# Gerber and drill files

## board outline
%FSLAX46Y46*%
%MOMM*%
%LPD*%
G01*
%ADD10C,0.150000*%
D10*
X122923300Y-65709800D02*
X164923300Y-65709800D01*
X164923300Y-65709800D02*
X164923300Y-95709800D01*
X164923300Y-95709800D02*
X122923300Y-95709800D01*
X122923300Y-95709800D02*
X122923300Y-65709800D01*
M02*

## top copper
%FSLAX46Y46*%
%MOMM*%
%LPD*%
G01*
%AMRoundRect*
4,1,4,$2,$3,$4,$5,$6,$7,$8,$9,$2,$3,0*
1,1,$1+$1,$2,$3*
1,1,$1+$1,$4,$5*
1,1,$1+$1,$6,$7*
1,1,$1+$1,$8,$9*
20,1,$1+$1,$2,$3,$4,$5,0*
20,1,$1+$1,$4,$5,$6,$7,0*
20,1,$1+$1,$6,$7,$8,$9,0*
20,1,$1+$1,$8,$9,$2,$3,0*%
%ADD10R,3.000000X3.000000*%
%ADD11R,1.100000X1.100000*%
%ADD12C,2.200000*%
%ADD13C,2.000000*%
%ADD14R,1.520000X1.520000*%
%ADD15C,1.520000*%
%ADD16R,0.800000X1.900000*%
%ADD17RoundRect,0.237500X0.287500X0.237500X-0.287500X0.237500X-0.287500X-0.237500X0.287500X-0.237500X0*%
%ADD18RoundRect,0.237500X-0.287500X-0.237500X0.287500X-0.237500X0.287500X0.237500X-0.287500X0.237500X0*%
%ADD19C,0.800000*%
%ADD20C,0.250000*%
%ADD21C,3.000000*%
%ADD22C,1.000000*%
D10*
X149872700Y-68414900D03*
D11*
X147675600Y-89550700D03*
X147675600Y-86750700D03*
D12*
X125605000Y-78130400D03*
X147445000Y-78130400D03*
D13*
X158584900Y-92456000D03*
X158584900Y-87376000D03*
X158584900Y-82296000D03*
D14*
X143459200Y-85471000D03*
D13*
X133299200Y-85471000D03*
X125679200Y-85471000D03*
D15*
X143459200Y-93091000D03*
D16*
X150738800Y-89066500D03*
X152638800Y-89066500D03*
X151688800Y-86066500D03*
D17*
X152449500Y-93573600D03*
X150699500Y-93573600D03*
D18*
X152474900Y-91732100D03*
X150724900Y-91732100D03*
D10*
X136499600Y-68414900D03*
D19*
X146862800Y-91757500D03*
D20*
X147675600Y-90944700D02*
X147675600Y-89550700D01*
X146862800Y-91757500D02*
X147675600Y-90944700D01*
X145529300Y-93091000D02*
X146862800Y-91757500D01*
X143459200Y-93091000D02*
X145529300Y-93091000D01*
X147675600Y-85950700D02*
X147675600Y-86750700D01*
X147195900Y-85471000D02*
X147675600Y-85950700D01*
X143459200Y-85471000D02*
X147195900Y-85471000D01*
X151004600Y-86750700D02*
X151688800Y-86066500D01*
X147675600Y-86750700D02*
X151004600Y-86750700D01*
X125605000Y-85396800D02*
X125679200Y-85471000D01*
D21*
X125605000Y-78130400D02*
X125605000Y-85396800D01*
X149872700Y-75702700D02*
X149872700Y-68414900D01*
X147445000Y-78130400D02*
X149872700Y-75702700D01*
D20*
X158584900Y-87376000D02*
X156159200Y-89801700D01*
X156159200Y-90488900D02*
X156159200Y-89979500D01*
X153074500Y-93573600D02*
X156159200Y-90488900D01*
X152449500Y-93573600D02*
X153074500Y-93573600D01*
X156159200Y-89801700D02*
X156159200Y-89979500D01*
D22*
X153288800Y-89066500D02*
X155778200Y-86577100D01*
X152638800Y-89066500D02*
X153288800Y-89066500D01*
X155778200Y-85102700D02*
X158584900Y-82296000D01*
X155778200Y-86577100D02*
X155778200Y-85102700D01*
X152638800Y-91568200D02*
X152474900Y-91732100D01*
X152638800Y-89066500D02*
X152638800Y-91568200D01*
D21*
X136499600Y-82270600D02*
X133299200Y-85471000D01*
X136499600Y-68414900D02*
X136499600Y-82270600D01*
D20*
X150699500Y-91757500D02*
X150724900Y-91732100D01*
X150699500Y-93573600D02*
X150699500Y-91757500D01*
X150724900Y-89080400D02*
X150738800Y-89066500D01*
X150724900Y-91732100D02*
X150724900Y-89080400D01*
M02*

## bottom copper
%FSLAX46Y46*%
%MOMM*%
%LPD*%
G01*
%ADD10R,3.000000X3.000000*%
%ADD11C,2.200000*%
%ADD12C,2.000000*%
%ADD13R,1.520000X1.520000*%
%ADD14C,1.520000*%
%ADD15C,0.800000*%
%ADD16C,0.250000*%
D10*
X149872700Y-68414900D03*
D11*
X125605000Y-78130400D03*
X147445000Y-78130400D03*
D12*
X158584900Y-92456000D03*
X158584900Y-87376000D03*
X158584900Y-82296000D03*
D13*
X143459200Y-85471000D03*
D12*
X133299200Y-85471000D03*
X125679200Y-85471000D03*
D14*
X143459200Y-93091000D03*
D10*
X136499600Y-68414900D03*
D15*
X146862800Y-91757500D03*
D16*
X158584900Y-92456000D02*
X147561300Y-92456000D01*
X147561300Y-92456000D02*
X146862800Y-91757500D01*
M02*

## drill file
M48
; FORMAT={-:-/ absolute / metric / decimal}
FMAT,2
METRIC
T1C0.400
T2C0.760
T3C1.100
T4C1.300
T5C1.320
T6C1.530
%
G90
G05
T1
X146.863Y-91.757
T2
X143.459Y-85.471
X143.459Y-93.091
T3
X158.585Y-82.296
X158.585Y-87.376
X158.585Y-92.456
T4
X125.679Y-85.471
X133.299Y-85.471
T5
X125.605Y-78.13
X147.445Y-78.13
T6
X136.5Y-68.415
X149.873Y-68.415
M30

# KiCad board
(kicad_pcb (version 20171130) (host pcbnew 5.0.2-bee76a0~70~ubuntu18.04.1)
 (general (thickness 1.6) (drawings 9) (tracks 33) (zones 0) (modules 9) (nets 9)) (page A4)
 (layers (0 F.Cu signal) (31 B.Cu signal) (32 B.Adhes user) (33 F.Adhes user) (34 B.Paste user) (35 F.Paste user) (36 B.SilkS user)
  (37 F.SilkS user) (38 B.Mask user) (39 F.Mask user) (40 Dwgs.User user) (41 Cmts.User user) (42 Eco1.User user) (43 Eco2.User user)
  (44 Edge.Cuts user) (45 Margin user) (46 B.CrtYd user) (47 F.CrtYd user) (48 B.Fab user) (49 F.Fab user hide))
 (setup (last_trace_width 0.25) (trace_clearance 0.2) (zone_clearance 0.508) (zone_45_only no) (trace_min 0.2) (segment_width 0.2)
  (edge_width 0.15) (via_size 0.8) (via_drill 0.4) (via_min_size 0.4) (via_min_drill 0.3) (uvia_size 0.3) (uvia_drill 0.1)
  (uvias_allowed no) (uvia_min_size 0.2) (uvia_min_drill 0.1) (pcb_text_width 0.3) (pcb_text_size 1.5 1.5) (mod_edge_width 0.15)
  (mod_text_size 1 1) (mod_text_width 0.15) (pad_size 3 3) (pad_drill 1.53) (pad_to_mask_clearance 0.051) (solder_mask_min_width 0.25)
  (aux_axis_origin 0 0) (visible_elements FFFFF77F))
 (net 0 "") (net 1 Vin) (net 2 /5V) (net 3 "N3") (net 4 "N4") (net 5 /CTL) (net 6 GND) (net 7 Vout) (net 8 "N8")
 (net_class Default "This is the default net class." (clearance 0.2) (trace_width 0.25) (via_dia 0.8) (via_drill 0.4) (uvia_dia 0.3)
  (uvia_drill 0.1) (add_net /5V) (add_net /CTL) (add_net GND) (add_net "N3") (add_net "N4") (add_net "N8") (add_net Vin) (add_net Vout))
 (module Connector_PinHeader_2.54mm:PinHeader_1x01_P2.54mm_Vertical (layer F.Cu) (at 149.8727 68.4149)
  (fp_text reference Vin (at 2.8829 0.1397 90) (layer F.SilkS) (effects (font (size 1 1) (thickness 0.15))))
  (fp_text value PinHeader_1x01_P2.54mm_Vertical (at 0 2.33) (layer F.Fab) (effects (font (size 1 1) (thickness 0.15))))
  (pad 1 thru_hole rect (at 0 0) (size 3 3) (drill 1.53) (layers *.Cu *.Mask) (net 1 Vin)))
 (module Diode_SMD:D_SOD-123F (layer F.Cu) (at 147.6756 88.1507 90)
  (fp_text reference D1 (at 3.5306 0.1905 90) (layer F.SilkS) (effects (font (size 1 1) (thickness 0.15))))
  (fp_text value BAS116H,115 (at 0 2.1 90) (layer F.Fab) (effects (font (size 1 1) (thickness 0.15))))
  (pad 1 smd rect (at -1.4 0 90) (size 1.1 1.1) (layers F.Cu F.Paste F.Mask) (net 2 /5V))
  (pad 2 smd rect (at 1.4 0 90) (size 1.1 1.1) (layers F.Cu F.Paste F.Mask) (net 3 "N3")))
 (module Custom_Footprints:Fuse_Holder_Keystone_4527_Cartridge (layer F.Cu) (at 136.525 78.1304)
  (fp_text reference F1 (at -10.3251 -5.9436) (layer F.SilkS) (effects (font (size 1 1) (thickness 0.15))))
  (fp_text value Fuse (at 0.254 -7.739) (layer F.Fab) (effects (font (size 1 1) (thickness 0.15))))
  (pad 1 thru_hole circle (at -10.92 0) (size 2.2 2.2) (drill 1.32) (layers *.Cu *.Mask) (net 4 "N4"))
  (pad 2 thru_hole circle (at 10.92 0) (size 2.2 2.2) (drill 1.32) (layers *.Cu *.Mask) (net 1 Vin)))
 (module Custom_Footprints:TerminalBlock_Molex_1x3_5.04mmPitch (layer F.Cu) (at 158.5849 87.376 90)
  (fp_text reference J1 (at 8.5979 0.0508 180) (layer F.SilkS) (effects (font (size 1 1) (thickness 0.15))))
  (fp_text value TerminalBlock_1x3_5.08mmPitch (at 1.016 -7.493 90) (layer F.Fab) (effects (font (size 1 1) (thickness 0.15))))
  (pad 1 thru_hole circle (at -5.08 0 90) (size 2 2) (drill 1.1) (layers *.Cu *.Mask) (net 2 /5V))
  (pad 2 thru_hole circle (at 0 0 90) (size 2 2) (drill 1.1) (layers *.Cu *.Mask) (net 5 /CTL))
  (pad 3 thru_hole circle (at 5.08 0 90) (size 2 2) (drill 1.1) (layers *.Cu *.Mask) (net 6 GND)))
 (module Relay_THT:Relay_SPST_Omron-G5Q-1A (layer F.Cu) (at 143.4592 85.471 180)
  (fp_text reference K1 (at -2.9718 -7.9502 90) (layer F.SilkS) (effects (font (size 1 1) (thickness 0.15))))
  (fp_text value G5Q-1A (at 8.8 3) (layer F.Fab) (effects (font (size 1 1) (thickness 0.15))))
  (pad 1 thru_hole rect (at 0 0) (size 1.52 1.52) (drill 0.76) (layers *.Cu *.Mask) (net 3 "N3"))
  (pad 2 thru_hole circle (at 10.16 0) (size 2 2) (drill 1.3) (layers *.Cu *.Mask) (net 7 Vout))
  (pad 3 thru_hole circle (at 17.78 0) (size 2 2) (drill 1.3) (layers *.Cu *.Mask) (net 4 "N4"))
  (pad 5 thru_hole circle (at 0 -7.62) (size 1.52 1.52) (drill 0.76) (layers *.Cu *.Mask) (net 2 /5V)))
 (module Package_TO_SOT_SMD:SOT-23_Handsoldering (layer F.Cu) (at 151.6888 87.5665 90)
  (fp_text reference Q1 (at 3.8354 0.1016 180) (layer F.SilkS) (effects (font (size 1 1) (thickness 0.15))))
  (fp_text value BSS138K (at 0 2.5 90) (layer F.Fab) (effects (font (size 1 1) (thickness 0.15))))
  (pad 1 smd rect (at -1.5 -0.95 90) (size 1.9 0.8) (layers F.Cu F.Paste F.Mask) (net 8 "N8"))
  (pad 2 smd rect (at -1.5 0.95 90) (size 1.9 0.8) (layers F.Cu F.Paste F.Mask) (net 6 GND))
  (pad 3 smd rect (at 1.5 0 90) (size 1.9 0.8) (layers F.Cu F.Paste F.Mask) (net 3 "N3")))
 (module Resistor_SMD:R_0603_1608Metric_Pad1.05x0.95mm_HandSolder (layer F.Cu) (at 151.5745 93.5736 180)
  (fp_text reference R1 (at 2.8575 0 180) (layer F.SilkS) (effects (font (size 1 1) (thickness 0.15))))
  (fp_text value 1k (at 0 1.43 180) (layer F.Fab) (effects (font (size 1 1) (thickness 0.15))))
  (pad 1 smd roundrect (at -0.875 0 180) (size 1.05 0.95) (layers F.Cu F.Paste F.Mask) (roundrect_rratio 0.25) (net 5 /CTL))
  (pad 2 smd roundrect (at 0.875 0 180) (size 1.05 0.95) (layers F.Cu F.Paste F.Mask) (roundrect_rratio 0.25) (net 8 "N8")))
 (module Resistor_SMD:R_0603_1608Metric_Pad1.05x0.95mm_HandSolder (layer F.Cu) (at 151.5999 91.7321)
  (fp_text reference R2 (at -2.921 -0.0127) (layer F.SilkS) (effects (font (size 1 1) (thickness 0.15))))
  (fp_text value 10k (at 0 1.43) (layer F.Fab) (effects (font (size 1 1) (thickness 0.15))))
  (pad 2 smd roundrect (at 0.875 0) (size 1.05 0.95) (layers F.Cu F.Paste F.Mask) (roundrect_rratio 0.25) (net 6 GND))
  (pad 1 smd roundrect (at -0.875 0) (size 1.05 0.95) (layers F.Cu F.Paste F.Mask) (roundrect_rratio 0.25) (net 8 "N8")))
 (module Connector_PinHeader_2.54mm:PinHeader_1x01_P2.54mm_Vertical (layer F.Cu) (at 136.4996 68.4149)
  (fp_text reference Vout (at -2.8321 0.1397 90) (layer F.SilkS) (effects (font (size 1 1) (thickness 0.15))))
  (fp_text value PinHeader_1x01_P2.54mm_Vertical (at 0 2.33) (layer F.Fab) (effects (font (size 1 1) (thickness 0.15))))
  (pad 1 thru_hole rect (at 0 0) (size 3 3) (drill 1.53) (layers *.Cu *.Mask) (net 7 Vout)))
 (gr_line (start 122.9233 65.7098) (end 164.9233 65.7098) (layer Edge.Cuts) (width 0.15))
 (gr_line (start 164.9233 65.7098) (end 164.9233 95.7098) (layer Edge.Cuts) (width 0.15))
 (gr_line (start 164.9233 95.7098) (end 122.9233 95.7098) (layer Edge.Cuts) (width 0.15))
 (gr_line (start 122.9233 95.7098) (end 122.9233 65.7098) (layer Edge.Cuts) (width 0.15))
 (via (at 146.8628 91.7575) (size 0.8) (drill 0.4) (layers F.Cu B.Cu) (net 2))
 (segment (start 158.5849 92.456) (end 147.5613 92.456) (width 0.25) (layer B.Cu) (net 2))
 (segment (start 147.5613 92.456) (end 146.8628 91.7575) (width 0.25) (layer B.Cu) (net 2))
 (segment (start 147.6756 90.9447) (end 147.6756 89.5507) (width 0.25) (layer F.Cu) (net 2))
 (segment (start 146.8628 91.7575) (end 147.6756 90.9447) (width 0.25) (layer F.Cu) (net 2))
 (segment (start 145.5293 93.091) (end 146.8628 91.7575) (width 0.25) (layer F.Cu) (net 2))
 (segment (start 143.4592 93.091) (end 145.5293 93.091) (width 0.25) (layer F.Cu) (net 2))
 (segment (start 147.6756 85.9507) (end 147.6756 86.7507) (width 0.25) (layer F.Cu) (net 3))
 (segment (start 147.1959 85.471) (end 147.6756 85.9507) (width 0.25) (layer F.Cu) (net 3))
 (segment (start 143.4592 85.471) (end 147.1959 85.471) (width 0.25) (layer F.Cu) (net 3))
 (segment (start 151.0046 86.7507) (end 151.6888 86.0665) (width 0.25) (layer F.Cu) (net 3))
 (segment (start 147.6756 86.7507) (end 151.0046 86.7507) (width 0.25) (layer F.Cu) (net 3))
 (segment (start 125.605 85.3968) (end 125.6792 85.471) (width 0.25) (layer F.Cu) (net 4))
 (segment (start 125.605 78.1304) (end 125.605 85.3968) (width 3) (layer F.Cu) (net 4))
 (segment (start 149.8727 75.7027) (end 149.8727 68.4149) (width 3) (layer F.Cu) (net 1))
 (segment (start 147.445 78.1304) (end 149.8727 75.7027) (width 3) (layer F.Cu) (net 1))
 (segment (start 158.5849 87.376) (end 156.1592 89.8017) (width 0.25) (layer F.Cu) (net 5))
 (segment (start 156.1592 90.4889) (end 156.1592 89.9795) (width 0.25) (layer F.Cu) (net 5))
 (segment (start 153.0745 93.5736) (end 156.1592 90.4889) (width 0.25) (layer F.Cu) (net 5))
 (segment (start 152.4495 93.5736) (end 153.0745 93.5736) (width 0.25) (layer F.Cu) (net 5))
 (segment (start 156.1592 89.8017) (end 156.1592 89.9795) (width 0.25) (layer F.Cu) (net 5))
 (segment (start 153.2888 89.0665) (end 155.7782 86.5771) (width 1) (layer F.Cu) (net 6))
 (segment (start 152.6388 89.0665) (end 153.2888 89.0665) (width 1) (layer F.Cu) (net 6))
 (segment (start 155.7782 85.1027) (end 158.5849 82.296) (width 1) (layer F.Cu) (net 6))
 (segment (start 155.7782 86.5771) (end 155.7782 85.1027) (width 1) (layer F.Cu) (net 6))
 (segment (start 152.6388 91.5682) (end 152.4749 91.7321) (width 1) (layer F.Cu) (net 6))
 (segment (start 152.6388 89.0665) (end 152.6388 91.5682) (width 1) (layer F.Cu) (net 6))
 (segment (start 136.4996 82.2706) (end 133.2992 85.471) (width 3) (layer F.Cu) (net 7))
 (segment (start 136.4996 68.4149) (end 136.4996 82.2706) (width 3) (layer F.Cu) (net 7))
 (segment (start 150.6995 91.7575) (end 150.7249 91.7321) (width 0.25) (layer F.Cu) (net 8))
 (segment (start 150.6995 93.5736) (end 150.6995 91.7575) (width 0.25) (layer F.Cu) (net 8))
 (segment (start 150.7249 89.0804) (end 150.7388 89.0665) (width 0.25) (layer F.Cu) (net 8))
 (segment (start 150.7249 91.7321) (end 150.7249 89.0804) (width 0.25) (layer F.Cu) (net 8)))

